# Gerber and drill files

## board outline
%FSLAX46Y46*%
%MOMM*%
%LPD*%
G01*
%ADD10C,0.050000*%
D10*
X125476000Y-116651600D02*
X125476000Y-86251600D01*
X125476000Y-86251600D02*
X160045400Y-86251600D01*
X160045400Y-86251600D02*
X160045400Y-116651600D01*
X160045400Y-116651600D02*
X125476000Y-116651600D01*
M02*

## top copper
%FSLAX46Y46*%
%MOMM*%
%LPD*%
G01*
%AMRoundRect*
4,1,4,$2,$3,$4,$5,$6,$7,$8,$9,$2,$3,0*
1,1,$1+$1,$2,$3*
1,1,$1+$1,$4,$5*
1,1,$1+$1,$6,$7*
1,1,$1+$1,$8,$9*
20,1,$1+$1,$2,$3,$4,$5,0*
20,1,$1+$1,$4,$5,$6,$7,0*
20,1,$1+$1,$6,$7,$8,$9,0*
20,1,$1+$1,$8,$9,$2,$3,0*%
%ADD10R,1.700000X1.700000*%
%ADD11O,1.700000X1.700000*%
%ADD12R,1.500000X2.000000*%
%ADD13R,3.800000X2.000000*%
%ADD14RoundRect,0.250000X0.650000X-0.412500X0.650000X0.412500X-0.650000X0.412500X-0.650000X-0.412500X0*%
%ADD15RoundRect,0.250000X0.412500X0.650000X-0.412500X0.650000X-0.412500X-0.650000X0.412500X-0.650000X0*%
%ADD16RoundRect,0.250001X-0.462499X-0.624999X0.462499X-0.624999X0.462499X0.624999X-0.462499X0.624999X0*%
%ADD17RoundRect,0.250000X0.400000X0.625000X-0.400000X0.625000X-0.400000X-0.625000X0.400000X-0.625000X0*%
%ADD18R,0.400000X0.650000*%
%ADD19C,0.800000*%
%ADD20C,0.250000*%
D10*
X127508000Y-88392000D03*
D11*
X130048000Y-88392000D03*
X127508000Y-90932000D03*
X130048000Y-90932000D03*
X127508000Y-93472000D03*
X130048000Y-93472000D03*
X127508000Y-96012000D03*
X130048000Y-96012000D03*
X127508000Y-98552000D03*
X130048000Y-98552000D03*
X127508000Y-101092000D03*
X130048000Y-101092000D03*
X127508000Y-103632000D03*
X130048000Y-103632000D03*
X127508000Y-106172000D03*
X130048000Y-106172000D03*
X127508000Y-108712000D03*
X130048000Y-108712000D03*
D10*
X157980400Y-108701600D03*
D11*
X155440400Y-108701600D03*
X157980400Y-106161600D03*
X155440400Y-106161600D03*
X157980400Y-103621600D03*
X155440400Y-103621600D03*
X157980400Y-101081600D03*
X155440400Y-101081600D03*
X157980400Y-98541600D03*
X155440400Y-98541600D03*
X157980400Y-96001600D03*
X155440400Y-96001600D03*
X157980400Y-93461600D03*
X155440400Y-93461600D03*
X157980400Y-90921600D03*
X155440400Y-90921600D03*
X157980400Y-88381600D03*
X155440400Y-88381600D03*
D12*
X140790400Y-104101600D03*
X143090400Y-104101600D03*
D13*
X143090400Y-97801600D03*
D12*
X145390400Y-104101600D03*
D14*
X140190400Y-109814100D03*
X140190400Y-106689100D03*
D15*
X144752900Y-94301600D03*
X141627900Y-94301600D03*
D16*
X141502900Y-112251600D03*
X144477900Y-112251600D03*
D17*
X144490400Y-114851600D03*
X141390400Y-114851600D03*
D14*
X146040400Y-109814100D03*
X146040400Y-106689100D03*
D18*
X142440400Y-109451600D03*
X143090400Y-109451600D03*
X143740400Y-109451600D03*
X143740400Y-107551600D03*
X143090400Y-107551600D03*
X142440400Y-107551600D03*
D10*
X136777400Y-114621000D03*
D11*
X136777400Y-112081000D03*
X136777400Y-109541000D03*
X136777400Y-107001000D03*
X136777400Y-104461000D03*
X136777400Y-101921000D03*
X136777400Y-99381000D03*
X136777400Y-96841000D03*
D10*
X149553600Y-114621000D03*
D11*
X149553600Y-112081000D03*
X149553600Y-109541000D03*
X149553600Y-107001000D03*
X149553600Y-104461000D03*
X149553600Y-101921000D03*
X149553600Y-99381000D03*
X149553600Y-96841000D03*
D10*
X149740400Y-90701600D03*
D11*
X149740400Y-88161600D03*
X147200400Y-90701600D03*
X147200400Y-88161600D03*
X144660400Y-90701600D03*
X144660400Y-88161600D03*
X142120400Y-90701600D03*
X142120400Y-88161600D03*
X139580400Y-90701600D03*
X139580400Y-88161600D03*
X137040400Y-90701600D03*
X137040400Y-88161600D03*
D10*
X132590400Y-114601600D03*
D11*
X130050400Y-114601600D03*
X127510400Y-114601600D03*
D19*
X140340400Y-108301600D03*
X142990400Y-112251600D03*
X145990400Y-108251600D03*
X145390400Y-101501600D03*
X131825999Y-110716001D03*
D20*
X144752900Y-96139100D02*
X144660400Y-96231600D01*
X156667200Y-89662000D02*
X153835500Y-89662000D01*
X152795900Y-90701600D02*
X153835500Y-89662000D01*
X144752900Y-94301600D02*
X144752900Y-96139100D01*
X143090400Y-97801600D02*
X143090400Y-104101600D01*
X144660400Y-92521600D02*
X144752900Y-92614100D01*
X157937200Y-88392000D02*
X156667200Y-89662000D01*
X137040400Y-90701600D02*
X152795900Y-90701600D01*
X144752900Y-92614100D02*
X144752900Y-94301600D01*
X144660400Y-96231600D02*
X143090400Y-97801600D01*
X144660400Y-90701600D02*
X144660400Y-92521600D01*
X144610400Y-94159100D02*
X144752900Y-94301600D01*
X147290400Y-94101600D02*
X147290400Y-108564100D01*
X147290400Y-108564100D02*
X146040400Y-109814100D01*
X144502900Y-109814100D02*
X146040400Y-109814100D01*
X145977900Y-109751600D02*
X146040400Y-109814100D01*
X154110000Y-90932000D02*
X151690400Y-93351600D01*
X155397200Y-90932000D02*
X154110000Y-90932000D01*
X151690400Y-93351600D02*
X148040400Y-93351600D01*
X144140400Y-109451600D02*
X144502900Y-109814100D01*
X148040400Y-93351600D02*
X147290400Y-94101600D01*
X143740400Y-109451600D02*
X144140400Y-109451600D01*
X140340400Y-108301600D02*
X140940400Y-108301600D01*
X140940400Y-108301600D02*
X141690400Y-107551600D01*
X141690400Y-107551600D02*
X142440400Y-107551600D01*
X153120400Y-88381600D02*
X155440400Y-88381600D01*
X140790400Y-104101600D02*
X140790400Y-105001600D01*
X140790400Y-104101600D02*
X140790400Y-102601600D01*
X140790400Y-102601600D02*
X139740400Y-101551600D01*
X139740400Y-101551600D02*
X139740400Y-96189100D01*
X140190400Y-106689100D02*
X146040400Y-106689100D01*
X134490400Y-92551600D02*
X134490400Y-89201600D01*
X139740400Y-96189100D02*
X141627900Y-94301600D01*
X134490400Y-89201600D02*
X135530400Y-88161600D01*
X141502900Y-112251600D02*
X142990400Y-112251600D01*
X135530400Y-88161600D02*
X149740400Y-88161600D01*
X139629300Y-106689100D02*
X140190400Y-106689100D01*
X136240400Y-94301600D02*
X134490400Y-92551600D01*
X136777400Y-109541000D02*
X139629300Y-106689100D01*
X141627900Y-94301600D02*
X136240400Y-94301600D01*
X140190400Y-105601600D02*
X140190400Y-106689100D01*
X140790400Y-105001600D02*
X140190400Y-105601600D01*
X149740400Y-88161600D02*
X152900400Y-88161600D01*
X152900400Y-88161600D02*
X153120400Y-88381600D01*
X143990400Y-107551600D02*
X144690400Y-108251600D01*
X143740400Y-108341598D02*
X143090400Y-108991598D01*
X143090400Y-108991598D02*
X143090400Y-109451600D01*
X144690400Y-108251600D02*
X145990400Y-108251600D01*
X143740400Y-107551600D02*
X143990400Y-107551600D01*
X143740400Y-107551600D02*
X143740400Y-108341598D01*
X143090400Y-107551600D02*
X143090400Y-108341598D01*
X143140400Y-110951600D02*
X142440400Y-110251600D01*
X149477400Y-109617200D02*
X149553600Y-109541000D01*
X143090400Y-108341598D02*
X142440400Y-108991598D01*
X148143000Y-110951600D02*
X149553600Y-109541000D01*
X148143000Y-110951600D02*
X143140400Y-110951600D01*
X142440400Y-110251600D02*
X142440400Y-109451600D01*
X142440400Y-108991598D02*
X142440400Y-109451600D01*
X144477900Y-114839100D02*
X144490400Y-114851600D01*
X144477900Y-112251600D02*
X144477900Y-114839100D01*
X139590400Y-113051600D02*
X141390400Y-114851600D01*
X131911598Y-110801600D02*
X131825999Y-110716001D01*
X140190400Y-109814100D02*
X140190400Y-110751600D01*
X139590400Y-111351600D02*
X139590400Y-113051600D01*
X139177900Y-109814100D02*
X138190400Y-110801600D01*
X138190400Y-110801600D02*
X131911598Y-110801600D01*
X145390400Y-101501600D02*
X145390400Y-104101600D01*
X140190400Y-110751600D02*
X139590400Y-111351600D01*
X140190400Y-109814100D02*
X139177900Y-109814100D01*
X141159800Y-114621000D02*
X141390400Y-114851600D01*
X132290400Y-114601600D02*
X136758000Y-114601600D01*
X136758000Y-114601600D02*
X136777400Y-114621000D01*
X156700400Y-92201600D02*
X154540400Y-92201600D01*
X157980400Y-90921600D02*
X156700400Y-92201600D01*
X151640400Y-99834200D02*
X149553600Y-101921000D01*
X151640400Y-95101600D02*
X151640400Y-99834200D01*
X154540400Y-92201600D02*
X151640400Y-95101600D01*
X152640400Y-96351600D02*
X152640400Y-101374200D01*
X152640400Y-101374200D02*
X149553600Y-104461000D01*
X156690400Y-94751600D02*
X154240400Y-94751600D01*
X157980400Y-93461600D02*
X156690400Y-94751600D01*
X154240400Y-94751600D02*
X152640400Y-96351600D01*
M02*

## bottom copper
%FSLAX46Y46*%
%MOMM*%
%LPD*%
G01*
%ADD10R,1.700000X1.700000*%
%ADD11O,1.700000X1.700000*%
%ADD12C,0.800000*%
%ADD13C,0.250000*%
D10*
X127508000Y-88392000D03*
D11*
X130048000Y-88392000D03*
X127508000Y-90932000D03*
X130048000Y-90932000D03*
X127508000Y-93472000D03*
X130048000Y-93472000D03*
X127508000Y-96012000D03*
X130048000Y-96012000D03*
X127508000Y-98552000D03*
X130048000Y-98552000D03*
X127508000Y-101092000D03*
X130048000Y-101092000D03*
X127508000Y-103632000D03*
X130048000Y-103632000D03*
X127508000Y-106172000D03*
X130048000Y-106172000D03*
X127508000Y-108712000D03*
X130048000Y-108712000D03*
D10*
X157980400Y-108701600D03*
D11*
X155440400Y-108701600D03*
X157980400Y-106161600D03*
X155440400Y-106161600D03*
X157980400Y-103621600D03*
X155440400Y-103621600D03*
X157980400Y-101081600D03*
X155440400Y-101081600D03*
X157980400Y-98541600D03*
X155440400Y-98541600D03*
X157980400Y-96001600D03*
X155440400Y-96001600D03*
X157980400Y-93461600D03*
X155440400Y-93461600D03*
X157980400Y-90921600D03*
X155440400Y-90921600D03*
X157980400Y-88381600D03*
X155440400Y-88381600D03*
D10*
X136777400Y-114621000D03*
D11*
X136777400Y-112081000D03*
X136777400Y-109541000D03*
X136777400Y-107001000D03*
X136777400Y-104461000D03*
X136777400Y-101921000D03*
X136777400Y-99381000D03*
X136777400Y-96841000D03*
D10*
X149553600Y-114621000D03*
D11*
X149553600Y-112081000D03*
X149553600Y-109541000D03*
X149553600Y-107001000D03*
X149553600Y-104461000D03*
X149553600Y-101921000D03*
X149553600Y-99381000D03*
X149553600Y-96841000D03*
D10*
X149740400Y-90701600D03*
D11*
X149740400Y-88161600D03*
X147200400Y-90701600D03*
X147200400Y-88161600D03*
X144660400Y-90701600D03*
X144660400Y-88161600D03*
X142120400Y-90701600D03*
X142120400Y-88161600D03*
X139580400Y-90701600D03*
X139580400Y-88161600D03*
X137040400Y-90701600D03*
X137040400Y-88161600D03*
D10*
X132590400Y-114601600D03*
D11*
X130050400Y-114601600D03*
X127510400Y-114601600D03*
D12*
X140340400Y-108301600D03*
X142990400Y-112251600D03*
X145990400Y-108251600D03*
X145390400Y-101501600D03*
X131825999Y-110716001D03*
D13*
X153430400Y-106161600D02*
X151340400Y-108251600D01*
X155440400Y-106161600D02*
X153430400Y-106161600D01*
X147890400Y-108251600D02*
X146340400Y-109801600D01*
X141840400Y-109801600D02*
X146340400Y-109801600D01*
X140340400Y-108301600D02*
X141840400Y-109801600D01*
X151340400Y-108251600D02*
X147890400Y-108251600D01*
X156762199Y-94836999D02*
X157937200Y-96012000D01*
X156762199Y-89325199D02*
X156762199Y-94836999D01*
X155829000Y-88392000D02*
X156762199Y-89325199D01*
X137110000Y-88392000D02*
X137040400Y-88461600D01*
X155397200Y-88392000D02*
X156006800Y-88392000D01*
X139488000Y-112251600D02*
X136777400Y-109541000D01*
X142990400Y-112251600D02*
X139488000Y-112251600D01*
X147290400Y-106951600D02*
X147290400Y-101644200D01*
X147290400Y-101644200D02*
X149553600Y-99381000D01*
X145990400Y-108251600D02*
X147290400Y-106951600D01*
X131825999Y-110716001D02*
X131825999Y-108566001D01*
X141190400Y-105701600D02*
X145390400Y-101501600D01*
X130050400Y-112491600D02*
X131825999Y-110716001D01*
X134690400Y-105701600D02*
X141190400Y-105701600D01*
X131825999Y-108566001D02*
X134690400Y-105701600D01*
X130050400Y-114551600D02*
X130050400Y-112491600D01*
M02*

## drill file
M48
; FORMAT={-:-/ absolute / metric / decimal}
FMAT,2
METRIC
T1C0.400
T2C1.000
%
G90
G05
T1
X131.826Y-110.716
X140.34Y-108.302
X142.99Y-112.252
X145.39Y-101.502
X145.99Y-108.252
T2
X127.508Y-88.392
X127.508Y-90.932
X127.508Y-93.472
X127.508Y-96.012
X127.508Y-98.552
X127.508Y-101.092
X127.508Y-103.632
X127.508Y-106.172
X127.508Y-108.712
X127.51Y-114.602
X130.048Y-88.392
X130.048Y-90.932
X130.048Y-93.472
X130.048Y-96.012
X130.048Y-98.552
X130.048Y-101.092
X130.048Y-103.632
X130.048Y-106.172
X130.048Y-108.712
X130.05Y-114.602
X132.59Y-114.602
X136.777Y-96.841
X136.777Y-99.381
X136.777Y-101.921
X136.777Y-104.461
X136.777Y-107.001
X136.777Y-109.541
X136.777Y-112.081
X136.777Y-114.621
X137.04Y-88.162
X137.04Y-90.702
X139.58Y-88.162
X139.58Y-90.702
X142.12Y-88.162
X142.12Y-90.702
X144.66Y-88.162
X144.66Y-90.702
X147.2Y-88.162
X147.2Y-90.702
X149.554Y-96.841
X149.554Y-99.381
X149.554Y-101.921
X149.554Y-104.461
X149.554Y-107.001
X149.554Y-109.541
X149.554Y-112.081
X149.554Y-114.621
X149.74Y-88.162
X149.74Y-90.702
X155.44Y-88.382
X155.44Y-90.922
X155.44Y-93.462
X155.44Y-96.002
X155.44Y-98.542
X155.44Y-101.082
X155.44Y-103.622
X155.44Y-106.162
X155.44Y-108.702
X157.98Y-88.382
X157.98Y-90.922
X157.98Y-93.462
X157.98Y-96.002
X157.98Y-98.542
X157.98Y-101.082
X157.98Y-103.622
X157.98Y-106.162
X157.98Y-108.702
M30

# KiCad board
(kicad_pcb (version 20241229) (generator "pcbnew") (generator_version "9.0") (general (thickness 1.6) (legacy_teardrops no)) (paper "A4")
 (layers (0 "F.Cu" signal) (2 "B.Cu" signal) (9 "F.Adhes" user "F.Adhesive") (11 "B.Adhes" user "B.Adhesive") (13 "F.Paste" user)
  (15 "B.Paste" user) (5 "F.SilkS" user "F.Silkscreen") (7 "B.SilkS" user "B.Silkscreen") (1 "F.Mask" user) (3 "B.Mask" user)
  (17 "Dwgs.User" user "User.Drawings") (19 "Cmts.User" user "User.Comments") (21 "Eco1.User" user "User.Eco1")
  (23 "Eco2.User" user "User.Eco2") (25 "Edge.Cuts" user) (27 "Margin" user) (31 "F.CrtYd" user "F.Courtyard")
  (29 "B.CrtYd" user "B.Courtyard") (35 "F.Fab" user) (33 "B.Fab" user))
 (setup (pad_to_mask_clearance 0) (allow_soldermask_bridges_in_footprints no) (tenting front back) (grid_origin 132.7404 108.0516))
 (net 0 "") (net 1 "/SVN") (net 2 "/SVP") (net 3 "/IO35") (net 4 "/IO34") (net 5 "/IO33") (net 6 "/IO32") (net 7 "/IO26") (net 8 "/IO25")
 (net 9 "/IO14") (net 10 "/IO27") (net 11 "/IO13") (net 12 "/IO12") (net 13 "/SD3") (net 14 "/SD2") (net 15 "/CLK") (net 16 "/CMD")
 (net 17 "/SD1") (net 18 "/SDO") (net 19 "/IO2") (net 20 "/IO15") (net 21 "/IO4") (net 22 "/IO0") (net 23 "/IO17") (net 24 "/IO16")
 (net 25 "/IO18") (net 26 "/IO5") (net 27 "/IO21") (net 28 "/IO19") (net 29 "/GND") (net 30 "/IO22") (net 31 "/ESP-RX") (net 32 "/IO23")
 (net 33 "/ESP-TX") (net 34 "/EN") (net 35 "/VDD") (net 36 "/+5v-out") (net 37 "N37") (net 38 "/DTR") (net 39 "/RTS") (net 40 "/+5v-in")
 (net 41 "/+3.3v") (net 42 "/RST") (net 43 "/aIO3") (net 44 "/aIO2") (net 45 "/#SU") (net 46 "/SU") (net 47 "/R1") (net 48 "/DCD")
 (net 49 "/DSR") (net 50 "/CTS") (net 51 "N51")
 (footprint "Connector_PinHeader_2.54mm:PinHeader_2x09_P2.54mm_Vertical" (layer "F.Cu") (at 127.508 88.392)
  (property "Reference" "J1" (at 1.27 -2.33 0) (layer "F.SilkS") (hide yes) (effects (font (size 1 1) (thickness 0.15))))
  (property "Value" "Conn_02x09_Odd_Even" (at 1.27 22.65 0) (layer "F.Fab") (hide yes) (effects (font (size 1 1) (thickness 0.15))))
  (pad "1" thru_hole rect (at 0 0) (size 1.7 1.7) (drill 1) (layers "*.Cu" "*.Mask") (remove_unused_layers no) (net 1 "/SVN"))
  (pad "2" thru_hole oval (at 2.54 0) (size 1.7 1.7) (drill 1) (layers "*.Cu" "*.Mask") (remove_unused_layers no) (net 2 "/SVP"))
  (pad "3" thru_hole oval (at 0 2.54) (size 1.7 1.7) (drill 1) (layers "*.Cu" "*.Mask") (remove_unused_layers no) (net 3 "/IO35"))
  (pad "4" thru_hole oval (at 2.54 2.54) (size 1.7 1.7) (drill 1) (layers "*.Cu" "*.Mask") (remove_unused_layers no) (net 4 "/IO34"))
  (pad "5" thru_hole oval (at 0 5.08) (size 1.7 1.7) (drill 1) (layers "*.Cu" "*.Mask") (remove_unused_layers no) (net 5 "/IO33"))
  (pad "6" thru_hole oval (at 2.54 5.08) (size 1.7 1.7) (drill 1) (layers "*.Cu" "*.Mask") (remove_unused_layers no) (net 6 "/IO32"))
  (pad "7" thru_hole oval (at 0 7.62) (size 1.7 1.7) (drill 1) (layers "*.Cu" "*.Mask") (remove_unused_layers no) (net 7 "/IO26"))
  (pad "8" thru_hole oval (at 2.54 7.62) (size 1.7 1.7) (drill 1) (layers "*.Cu" "*.Mask") (remove_unused_layers no) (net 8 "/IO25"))
  (pad "9" thru_hole oval (at 0 10.16) (size 1.7 1.7) (drill 1) (layers "*.Cu" "*.Mask") (remove_unused_layers no) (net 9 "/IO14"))
  (pad "10" thru_hole oval (at 2.54 10.16) (size 1.7 1.7) (drill 1) (layers "*.Cu" "*.Mask") (remove_unused_layers no) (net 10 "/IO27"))
  (pad "11" thru_hole oval (at 0 12.7) (size 1.7 1.7) (drill 1) (layers "*.Cu" "*.Mask") (remove_unused_layers no) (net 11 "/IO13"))
  (pad "12" thru_hole oval (at 2.54 12.7) (size 1.7 1.7) (drill 1) (layers "*.Cu" "*.Mask") (remove_unused_layers no) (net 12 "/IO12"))
  (pad "13" thru_hole oval (at 0 15.24) (size 1.7 1.7) (drill 1) (layers "*.Cu" "*.Mask") (remove_unused_layers no) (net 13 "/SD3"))
  (pad "14" thru_hole oval (at 2.54 15.24) (size 1.7 1.7) (drill 1) (layers "*.Cu" "*.Mask") (remove_unused_layers no) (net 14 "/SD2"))
  (pad "15" thru_hole oval (at 0 17.78) (size 1.7 1.7) (drill 1) (layers "*.Cu" "*.Mask") (remove_unused_layers no) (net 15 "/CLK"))
  (pad "16" thru_hole oval (at 2.54 17.78) (size 1.7 1.7) (drill 1) (layers "*.Cu" "*.Mask") (remove_unused_layers no) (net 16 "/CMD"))
  (pad "17" thru_hole oval (at 0 20.32) (size 1.7 1.7) (drill 1) (layers "*.Cu" "*.Mask") (remove_unused_layers no) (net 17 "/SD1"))
  (pad "18" thru_hole oval (at 2.54 20.32) (size 1.7 1.7) (drill 1) (layers "*.Cu" "*.Mask") (remove_unused_layers no) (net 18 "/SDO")))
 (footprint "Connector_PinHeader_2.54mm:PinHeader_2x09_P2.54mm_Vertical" (layer "F.Cu") (at 157.9804 108.7016 180)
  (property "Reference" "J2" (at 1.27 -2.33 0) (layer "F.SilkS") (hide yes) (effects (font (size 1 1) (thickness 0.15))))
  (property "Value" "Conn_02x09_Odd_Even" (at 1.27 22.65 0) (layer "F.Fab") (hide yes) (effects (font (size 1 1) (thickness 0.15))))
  (pad "1" thru_hole rect (at 0 0 180) (size 1.7 1.7) (drill 1) (layers "*.Cu" "*.Mask") (remove_unused_layers no) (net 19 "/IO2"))
  (pad "2" thru_hole oval (at 2.54 0 180) (size 1.7 1.7) (drill 1) (layers "*.Cu" "*.Mask") (remove_unused_layers no) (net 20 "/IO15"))
  (pad "3" thru_hole oval (at 0 2.54 180) (size 1.7 1.7) (drill 1) (layers "*.Cu" "*.Mask") (remove_unused_layers no) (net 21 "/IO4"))
  (pad "4" thru_hole oval (at 2.54 2.54 180) (size 1.7 1.7) (drill 1) (layers "*.Cu" "*.Mask") (remove_unused_layers no) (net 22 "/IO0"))
  (pad "5" thru_hole oval (at 0 5.08 180) (size 1.7 1.7) (drill 1) (layers "*.Cu" "*.Mask") (remove_unused_layers no) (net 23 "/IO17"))
  (pad "6" thru_hole oval (at 2.54 5.08 180) (size 1.7 1.7) (drill 1) (layers "*.Cu" "*.Mask") (remove_unused_layers no) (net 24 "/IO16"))
  (pad "7" thru_hole oval (at 0 7.62 180) (size 1.7 1.7) (drill 1) (layers "*.Cu" "*.Mask") (remove_unused_layers no) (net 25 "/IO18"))
  (pad "8" thru_hole oval (at 2.54 7.62 180) (size 1.7 1.7) (drill 1) (layers "*.Cu" "*.Mask") (remove_unused_layers no) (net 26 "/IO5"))
  (pad "9" thru_hole oval (at 0 10.16 180) (size 1.7 1.7) (drill 1) (layers "*.Cu" "*.Mask") (remove_unused_layers no) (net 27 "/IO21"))
  (pad "10" thru_hole oval (at 2.54 10.16 180) (size 1.7 1.7) (drill 1) (layers "*.Cu" "*.Mask") (remove_unused_layers no) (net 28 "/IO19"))
  (pad "11" thru_hole oval (at 0 12.7 180) (size 1.7 1.7) (drill 1) (layers "*.Cu" "*.Mask") (remove_unused_layers no) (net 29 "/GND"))
  (pad "12" thru_hole oval (at 2.54 12.7 180) (size 1.7 1.7) (drill 1) (layers "*.Cu" "*.Mask") (remove_unused_layers no) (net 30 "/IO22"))
  (pad "13" thru_hole oval (at 0 15.24 180) (size 1.7 1.7) (drill 1) (layers "*.Cu" "*.Mask") (remove_unused_layers no) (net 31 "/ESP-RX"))
  (pad "14" thru_hole oval (at 2.54 15.24 180) (size 1.7 1.7) (drill 1) (layers "*.Cu" "*.Mask") (remove_unused_layers no) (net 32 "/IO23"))
  (pad "15" thru_hole oval (at 0 17.78 180) (size 1.7 1.7) (drill 1) (layers "*.Cu" "*.Mask") (remove_unused_layers no) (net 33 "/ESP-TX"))
  (pad "16" thru_hole oval (at 2.54 17.78 180) (size 1.7 1.7) (drill 1) (layers "*.Cu" "*.Mask") (remove_unused_layers no) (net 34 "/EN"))
  (pad "17" thru_hole oval (at 0 20.32 180) (size 1.7 1.7) (drill 1) (layers "*.Cu" "*.Mask") (remove_unused_layers no) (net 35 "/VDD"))
  (pad "18" thru_hole oval (at 2.54 20.32 180) (size 1.7 1.7) (drill 1) (layers "*.Cu" "*.Mask") (remove_unused_layers no) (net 29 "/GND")))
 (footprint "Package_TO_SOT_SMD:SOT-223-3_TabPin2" (layer "F.Cu") (at 143.0904 100.9516 90)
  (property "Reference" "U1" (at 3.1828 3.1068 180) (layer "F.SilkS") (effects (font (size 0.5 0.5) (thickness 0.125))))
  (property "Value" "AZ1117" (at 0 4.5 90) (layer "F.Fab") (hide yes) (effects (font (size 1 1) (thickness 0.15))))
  (pad "1" smd rect (at -3.15 -2.3 90) (size 2 1.5) (layers "F.Cu" "F.Mask" "F.Paste") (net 29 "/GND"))
  (pad "2" smd rect (at -3.15 0 90) (size 2 1.5) (layers "F.Cu" "F.Mask" "F.Paste") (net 35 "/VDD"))
  (pad "2" smd rect (at 3.15 0 90) (size 2 3.8) (layers "F.Cu" "F.Mask" "F.Paste") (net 35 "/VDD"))
  (pad "3" smd rect (at -3.15 2.3 90) (size 2 1.5) (layers "F.Cu" "F.Mask" "F.Paste") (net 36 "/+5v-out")))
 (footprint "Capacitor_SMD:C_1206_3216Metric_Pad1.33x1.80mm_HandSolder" (layer "F.Cu") (at 140.1904 108.2516 90)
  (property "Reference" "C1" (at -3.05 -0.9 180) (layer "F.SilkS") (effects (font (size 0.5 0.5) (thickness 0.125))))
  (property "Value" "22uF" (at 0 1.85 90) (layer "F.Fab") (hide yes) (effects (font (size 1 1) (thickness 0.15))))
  (pad "1" smd roundrect (at -1.5625 0 90) (size 1.325 1.8) (layers "F.Cu" "F.Mask" "F.Paste") (roundrect_rratio 0.188679)
   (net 36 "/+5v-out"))
  (pad "2" smd roundrect (at 1.5625 0 90) (size 1.325 1.8) (layers "F.Cu" "F.Mask" "F.Paste") (roundrect_rratio 0.188679) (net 29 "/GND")))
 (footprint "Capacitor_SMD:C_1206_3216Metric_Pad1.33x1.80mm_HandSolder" (layer "F.Cu") (at 143.1904 94.3016 180)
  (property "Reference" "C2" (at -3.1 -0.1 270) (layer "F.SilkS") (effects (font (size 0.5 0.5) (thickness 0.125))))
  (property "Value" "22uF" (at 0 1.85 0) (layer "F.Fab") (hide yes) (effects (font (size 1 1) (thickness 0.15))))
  (pad "1" smd roundrect (at -1.5625 0 180) (size 1.325 1.8) (layers "F.Cu" "F.Mask" "F.Paste") (roundrect_rratio 0.188679) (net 35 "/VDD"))
  (pad "2" smd roundrect (at 1.5625 0 180) (size 1.325 1.8) (layers "F.Cu" "F.Mask" "F.Paste") (roundrect_rratio 0.188679) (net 29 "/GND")))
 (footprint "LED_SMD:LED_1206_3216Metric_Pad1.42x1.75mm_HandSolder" (layer "F.Cu") (at 142.9904 112.2516)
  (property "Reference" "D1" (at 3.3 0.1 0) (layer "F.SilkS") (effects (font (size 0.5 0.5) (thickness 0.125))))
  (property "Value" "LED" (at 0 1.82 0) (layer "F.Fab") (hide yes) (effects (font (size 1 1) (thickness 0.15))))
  (pad "1" smd roundrect (at -1.4875 0) (size 1.425 1.75) (layers "F.Cu" "F.Mask" "F.Paste") (roundrect_rratio 0.175439) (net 29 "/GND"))
  (pad "2" smd roundrect (at 1.4875 0) (size 1.425 1.75) (layers "F.Cu" "F.Mask" "F.Paste") (roundrect_rratio 0.175439) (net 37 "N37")))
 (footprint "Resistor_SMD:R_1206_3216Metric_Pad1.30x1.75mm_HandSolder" (layer "F.Cu") (at 142.9404 114.8516 180)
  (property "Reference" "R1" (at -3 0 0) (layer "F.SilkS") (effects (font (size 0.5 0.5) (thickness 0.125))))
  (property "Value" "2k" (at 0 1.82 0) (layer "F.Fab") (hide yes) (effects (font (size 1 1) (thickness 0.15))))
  (pad "1" smd roundrect (at -1.55 0 180) (size 1.3 1.75) (layers "F.Cu" "F.Mask" "F.Paste") (roundrect_rratio 0.192308) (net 37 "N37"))
  (pad "2" smd roundrect (at 1.55 0 180) (size 1.3 1.75) (layers "F.Cu" "F.Mask" "F.Paste") (roundrect_rratio 0.192308) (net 36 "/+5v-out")))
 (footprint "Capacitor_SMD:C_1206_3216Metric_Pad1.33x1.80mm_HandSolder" (layer "F.Cu") (at 146.0404 108.2516 90)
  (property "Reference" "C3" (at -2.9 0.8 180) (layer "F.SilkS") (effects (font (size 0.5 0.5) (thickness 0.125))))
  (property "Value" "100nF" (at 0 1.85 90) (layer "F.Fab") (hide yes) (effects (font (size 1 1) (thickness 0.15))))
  (pad "1" smd roundrect (at -1.5625 0 90) (size 1.325 1.8) (layers "F.Cu" "F.Mask" "F.Paste") (roundrect_rratio 0.188679) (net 34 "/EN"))
  (pad "2" smd roundrect (at 1.5625 0 90) (size 1.325 1.8) (layers "F.Cu" "F.Mask" "F.Paste") (roundrect_rratio 0.188679) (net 29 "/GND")))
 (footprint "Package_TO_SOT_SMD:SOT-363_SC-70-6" (layer "F.Cu") (at 143.0904 108.5016 90)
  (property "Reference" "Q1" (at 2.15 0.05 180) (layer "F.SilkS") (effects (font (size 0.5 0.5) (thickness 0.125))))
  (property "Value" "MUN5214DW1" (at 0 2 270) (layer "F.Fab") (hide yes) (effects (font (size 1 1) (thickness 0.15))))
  (pad "1" smd rect (at -0.95 -0.65 90) (size 0.65 0.4) (layers "F.Cu" "F.Mask" "F.Paste") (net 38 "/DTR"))
  (pad "2" smd rect (at -0.95 0 90) (size 0.65 0.4) (layers "F.Cu" "F.Mask" "F.Paste") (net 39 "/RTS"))
  (pad "3" smd rect (at -0.95 0.65 90) (size 0.65 0.4) (layers "F.Cu" "F.Mask" "F.Paste") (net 34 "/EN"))
  (pad "4" smd rect (at 0.95 0.65 90) (size 0.65 0.4) (layers "F.Cu" "F.Mask" "F.Paste") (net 39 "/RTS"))
  (pad "5" smd rect (at 0.95 0 90) (size 0.65 0.4) (layers "F.Cu" "F.Mask" "F.Paste") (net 38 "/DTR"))
  (pad "6" smd rect (at 0.95 -0.65 90) (size 0.65 0.4) (layers "F.Cu" "F.Mask" "F.Paste") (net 22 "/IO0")))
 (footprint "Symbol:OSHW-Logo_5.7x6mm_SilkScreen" (layer "B.Cu") (at 143.5404 95.6016 180)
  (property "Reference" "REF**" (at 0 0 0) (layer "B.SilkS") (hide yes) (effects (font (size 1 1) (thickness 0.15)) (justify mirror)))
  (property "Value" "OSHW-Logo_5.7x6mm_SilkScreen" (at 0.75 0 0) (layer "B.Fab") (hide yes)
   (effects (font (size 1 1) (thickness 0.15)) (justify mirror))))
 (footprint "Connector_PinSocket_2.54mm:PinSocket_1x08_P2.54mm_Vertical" (layer "B.Cu") (at 136.7774 114.621)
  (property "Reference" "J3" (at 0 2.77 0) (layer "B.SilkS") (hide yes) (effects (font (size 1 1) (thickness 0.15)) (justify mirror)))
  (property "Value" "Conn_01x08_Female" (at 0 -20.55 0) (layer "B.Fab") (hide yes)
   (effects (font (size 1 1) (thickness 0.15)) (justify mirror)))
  (pad "1" thru_hole rect (at 0 0) (size 1.7 1.7) (drill 1) (layers "*.Cu" "*.Mask") (remove_unused_layers no) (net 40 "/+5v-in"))
  (pad "2" thru_hole oval (at 0 -2.54) (size 1.7 1.7) (drill 1) (layers "*.Cu" "*.Mask") (remove_unused_layers no) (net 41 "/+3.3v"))
  (pad "3" thru_hole oval (at 0 -5.08) (size 1.7 1.7) (drill 1) (layers "*.Cu" "*.Mask") (remove_unused_layers no) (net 29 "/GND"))
  (pad "4" thru_hole oval (at 0 -7.62) (size 1.7 1.7) (drill 1) (layers "*.Cu" "*.Mask") (remove_unused_layers no) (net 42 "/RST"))
  (pad "5" thru_hole oval (at 0 -10.16) (size 1.7 1.7) (drill 1) (layers "*.Cu" "*.Mask") (remove_unused_layers no) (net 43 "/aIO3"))
  (pad "6" thru_hole oval (at 0 -12.7) (size 1.7 1.7) (drill 1) (layers "*.Cu" "*.Mask") (remove_unused_layers no) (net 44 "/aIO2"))
  (pad "7" thru_hole oval (at 0 -15.24) (size 1.7 1.7) (drill 1) (layers "*.Cu" "*.Mask") (remove_unused_layers no) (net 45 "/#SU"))
  (pad "8" thru_hole oval (at 0 -17.78) (size 1.7 1.7) (drill 1) (layers "*.Cu" "*.Mask") (remove_unused_layers no) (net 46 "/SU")))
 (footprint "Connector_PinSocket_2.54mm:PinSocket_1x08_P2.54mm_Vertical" (layer "B.Cu") (at 149.5536 114.621)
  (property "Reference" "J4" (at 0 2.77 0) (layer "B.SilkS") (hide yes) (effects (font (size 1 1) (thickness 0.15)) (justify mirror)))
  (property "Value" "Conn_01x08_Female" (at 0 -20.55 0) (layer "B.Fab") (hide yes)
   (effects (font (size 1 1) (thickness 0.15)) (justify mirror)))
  (pad "1" thru_hole rect (at 0 0) (size 1.7 1.7) (drill 1) (layers "*.Cu" "*.Mask") (remove_unused_layers no) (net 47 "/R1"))
  (pad "2" thru_hole oval (at 0 -2.54) (size 1.7 1.7) (drill 1) (layers "*.Cu" "*.Mask") (remove_unused_layers no) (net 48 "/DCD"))
  (pad "3" thru_hole oval (at 0 -5.08) (size 1.7 1.7) (drill 1) (layers "*.Cu" "*.Mask") (remove_unused_layers no) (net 38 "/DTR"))
  (pad "4" thru_hole oval (at 0 -7.62) (size 1.7 1.7) (drill 1) (layers "*.Cu" "*.Mask") (remove_unused_layers no) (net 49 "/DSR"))
  (pad "5" thru_hole oval (at 0 -10.16) (size 1.7 1.7) (drill 1) (layers "*.Cu" "*.Mask") (remove_unused_layers no) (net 31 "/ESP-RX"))
  (pad "6" thru_hole oval (at 0 -12.7) (size 1.7 1.7) (drill 1) (layers "*.Cu" "*.Mask") (remove_unused_layers no) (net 33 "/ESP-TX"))
  (pad "7" thru_hole oval (at 0 -15.24) (size 1.7 1.7) (drill 1) (layers "*.Cu" "*.Mask") (remove_unused_layers no) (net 39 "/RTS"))
  (pad "8" thru_hole oval (at 0 -17.78) (size 1.7 1.7) (drill 1) (layers "*.Cu" "*.Mask") (remove_unused_layers no) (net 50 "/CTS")))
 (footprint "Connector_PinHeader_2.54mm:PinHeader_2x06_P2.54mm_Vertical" (layer "B.Cu") (at 149.7404 90.7016 90)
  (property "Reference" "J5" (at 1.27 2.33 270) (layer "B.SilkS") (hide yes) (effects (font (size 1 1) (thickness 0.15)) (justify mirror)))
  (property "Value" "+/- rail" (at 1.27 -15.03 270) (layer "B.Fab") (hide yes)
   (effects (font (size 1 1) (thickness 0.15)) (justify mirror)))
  (pad "1" thru_hole rect (at 0 0 90) (size 1.7 1.7) (drill 1) (layers "*.Cu" "*.Mask") (remove_unused_layers no) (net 35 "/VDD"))
  (pad "2" thru_hole oval (at 2.54 0 90) (size 1.7 1.7) (drill 1) (layers "*.Cu" "*.Mask") (remove_unused_layers no) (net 29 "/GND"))
  (pad "3" thru_hole oval (at 0 -2.54 90) (size 1.7 1.7) (drill 1) (layers "*.Cu" "*.Mask") (remove_unused_layers no) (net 35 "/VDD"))
  (pad "4" thru_hole oval (at 2.54 -2.54 90) (size 1.7 1.7) (drill 1) (layers "*.Cu" "*.Mask") (remove_unused_layers no) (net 29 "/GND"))
  (pad "5" thru_hole oval (at 0 -5.08 90) (size 1.7 1.7) (drill 1) (layers "*.Cu" "*.Mask") (remove_unused_layers no) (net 35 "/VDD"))
  (pad "6" thru_hole oval (at 2.54 -5.08 90) (size 1.7 1.7) (drill 1) (layers "*.Cu" "*.Mask") (remove_unused_layers no) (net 29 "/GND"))
  (pad "7" thru_hole oval (at 0 -7.62 90) (size 1.7 1.7) (drill 1) (layers "*.Cu" "*.Mask") (remove_unused_layers no) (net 35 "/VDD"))
  (pad "8" thru_hole oval (at 2.54 -7.62 90) (size 1.7 1.7) (drill 1) (layers "*.Cu" "*.Mask") (remove_unused_layers no) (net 29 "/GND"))
  (pad "9" thru_hole oval (at 0 -10.16 90) (size 1.7 1.7) (drill 1) (layers "*.Cu" "*.Mask") (remove_unused_layers no) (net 35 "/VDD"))
  (pad "10" thru_hole oval (at 2.54 -10.16 90) (size 1.7 1.7) (drill 1) (layers "*.Cu" "*.Mask") (remove_unused_layers no) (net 29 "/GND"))
  (pad "11" thru_hole oval (at 0 -12.7 90) (size 1.7 1.7) (drill 1) (layers "*.Cu" "*.Mask") (remove_unused_layers no) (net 35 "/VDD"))
  (pad "12" thru_hole oval (at 2.54 -12.7 90) (size 1.7 1.7) (drill 1) (layers "*.Cu" "*.Mask") (remove_unused_layers no) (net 29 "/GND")))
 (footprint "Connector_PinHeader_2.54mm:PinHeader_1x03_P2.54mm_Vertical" (layer "B.Cu") (at 132.5904 114.6016 90)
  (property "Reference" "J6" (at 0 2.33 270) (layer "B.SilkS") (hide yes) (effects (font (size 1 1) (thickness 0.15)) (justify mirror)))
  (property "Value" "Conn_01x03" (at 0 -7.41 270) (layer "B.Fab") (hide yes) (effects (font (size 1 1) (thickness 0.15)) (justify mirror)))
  (pad "1" thru_hole rect (at 0 0 90) (size 1.7 1.7) (drill 1) (layers "*.Cu" "*.Mask") (remove_unused_layers no) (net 40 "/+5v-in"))
  (pad "2" thru_hole oval (at 0 -2.54 90) (size 1.7 1.7) (drill 1) (layers "*.Cu" "*.Mask") (remove_unused_layers no) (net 36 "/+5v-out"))
  (pad "3" thru_hole oval (at 0 -5.08 90) (size 1.7 1.7) (drill 1) (layers "*.Cu" "*.Mask") (remove_unused_layers no) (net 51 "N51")))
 (gr_line (start 125.476 116.6516) (end 125.476 86.2516) (stroke (width 0.05) (type solid)) (layer "Edge.Cuts"))
 (gr_line (start 125.476 86.2516) (end 160.0454 86.2516) (stroke (width 0.05) (type solid)) (layer "Edge.Cuts"))
 (gr_line (start 160.0454 86.2516) (end 160.0454 116.6516) (stroke (width 0.05) (type solid)) (layer "Edge.Cuts"))
 (gr_line (start 160.0454 116.6516) (end 125.476 116.6516) (stroke (width 0.05) (type solid)) (layer "Edge.Cuts"))
 (segment (start 144.7529 96.1391) (end 144.6604 96.2316) (width 0.25) (layer "F.Cu") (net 35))
 (segment (start 156.6672 89.662) (end 153.8355 89.662) (width 0.25) (layer "F.Cu") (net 35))
 (segment (start 152.7959 90.7016) (end 153.8355 89.662) (width 0.25) (layer "F.Cu") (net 35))
 (segment (start 144.7529 94.3016) (end 144.7529 96.1391) (width 0.25) (layer "F.Cu") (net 35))
 (segment (start 143.0904 97.8016) (end 143.0904 104.1016) (width 0.25) (layer "F.Cu") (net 35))
 (segment (start 144.6604 92.5216) (end 144.7529 92.6141) (width 0.25) (layer "F.Cu") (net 35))
 (segment (start 157.9372 88.392) (end 156.6672 89.662) (width 0.25) (layer "F.Cu") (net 35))
 (segment (start 137.0404 90.7016) (end 152.7959 90.7016) (width 0.25) (layer "F.Cu") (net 35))
 (segment (start 144.7529 92.6141) (end 144.7529 94.3016) (width 0.25) (layer "F.Cu") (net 35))
 (segment (start 144.6604 96.2316) (end 143.0904 97.8016) (width 0.25) (layer "F.Cu") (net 35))
 (segment (start 144.6604 90.7016) (end 144.6604 92.5216) (width 0.25) (layer "F.Cu") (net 35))
 (segment (start 144.6104 94.1591) (end 144.7529 94.3016) (width 0.25) (layer "F.Cu") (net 35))
 (segment (start 147.2904 94.1016) (end 147.2904 108.5641) (width 0.25) (layer "F.Cu") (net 34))
 (segment (start 147.2904 108.5641) (end 146.0404 109.8141) (width 0.25) (layer "F.Cu") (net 34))
 (segment (start 144.5029 109.8141) (end 146.0404 109.8141) (width 0.25) (layer "F.Cu") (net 34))
 (segment (start 145.9779 109.7516) (end 146.0404 109.8141) (width 0.25) (layer "F.Cu") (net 34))
 (segment (start 154.11 90.932) (end 151.6904 93.3516) (width 0.25) (layer "F.Cu") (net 34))
 (segment (start 155.3972 90.932) (end 154.11 90.932) (width 0.25) (layer "F.Cu") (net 34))
 (segment (start 151.6904 93.3516) (end 148.0404 93.3516) (width 0.25) (layer "F.Cu") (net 34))
 (segment (start 144.1404 109.4516) (end 144.5029 109.8141) (width 0.25) (layer "F.Cu") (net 34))
 (segment (start 148.0404 93.3516) (end 147.2904 94.1016) (width 0.25) (layer "F.Cu") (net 34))
 (segment (start 143.7404 109.4516) (end 144.1404 109.4516) (width 0.25) (layer "F.Cu") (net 34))
 (segment (start 140.3404 108.3016) (end 140.9404 108.3016) (width 0.25) (layer "F.Cu") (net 22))
 (segment (start 140.9404 108.3016) (end 141.6904 107.5516) (width 0.25) (layer "F.Cu") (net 22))
 (segment (start 141.6904 107.5516) (end 142.4404 107.5516) (width 0.25) (layer "F.Cu") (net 22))
 (via (at 140.3404 108.3016) (size 0.8) (drill 0.4) (layers "F.Cu" "B.Cu") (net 22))
 (segment (start 153.4304 106.1616) (end 151.3404 108.2516) (width 0.25) (layer "B.Cu") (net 22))
 (segment (start 155.4404 106.1616) (end 153.4304 106.1616) (width 0.25) (layer "B.Cu") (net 22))
 (segment (start 147.8904 108.2516) (end 146.3404 109.8016) (width 0.25) (layer "B.Cu") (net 22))
 (segment (start 141.8404 109.8016) (end 146.3404 109.8016) (width 0.25) (layer "B.Cu") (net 22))
 (segment (start 140.3404 108.3016) (end 141.8404 109.8016) (width 0.25) (layer "B.Cu") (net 22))
 (segment (start 151.3404 108.2516) (end 147.8904 108.2516) (width 0.25) (layer "B.Cu") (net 22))
 (segment (start 153.1204 88.3816) (end 155.4404 88.3816) (width 0.25) (layer "F.Cu") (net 29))
 (segment (start 140.7904 104.1016) (end 140.7904 105.0016) (width 0.25) (layer "F.Cu") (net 29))
 (segment (start 140.7904 104.1016) (end 140.7904 102.6016) (width 0.25) (layer "F.Cu") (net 29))
 (segment (start 140.7904 102.6016) (end 139.7404 101.5516) (width 0.25) (layer "F.Cu") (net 29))
 (segment (start 139.7404 101.5516) (end 139.7404 96.1891) (width 0.25) (layer "F.Cu") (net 29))
 (segment (start 140.1904 106.6891) (end 146.0404 106.6891) (width 0.25) (layer "F.Cu") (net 29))
 (segment (start 134.4904 92.5516) (end 134.4904 89.2016) (width 0.25) (layer "F.Cu") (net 29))
 (segment (start 139.7404 96.1891) (end 141.6279 94.3016) (width 0.25) (layer "F.Cu") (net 29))
 (segment (start 134.4904 89.2016) (end 135.5304 88.1616) (width 0.25) (layer "F.Cu") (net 29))
 (segment (start 141.5029 112.2516) (end 142.9904 112.2516) (width 0.25) (layer "F.Cu") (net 29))
 (segment (start 135.5304 88.1616) (end 149.7404 88.1616) (width 0.25) (layer "F.Cu") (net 29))
 (segment (start 139.6293 106.6891) (end 140.1904 106.6891) (width 0.25) (layer "F.Cu") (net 29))
 (segment (start 136.2404 94.3016) (end 134.4904 92.5516) (width 0.25) (layer "F.Cu") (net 29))
 (segment (start 136.7774 109.541) (end 139.6293 106.6891) (width 0.25) (layer "F.Cu") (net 29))
 (segment (start 141.6279 94.3016) (end 136.2404 94.3016) (width 0.25) (layer "F.Cu") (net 29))
 (segment (start 140.1904 105.6016) (end 140.1904 106.6891) (width 0.25) (layer "F.Cu") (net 29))
 (segment (start 140.7904 105.0016) (end 140.1904 105.6016) (width 0.25) (layer "F.Cu") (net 29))
 (segment (start 149.7404 88.1616) (end 152.9004 88.1616) (width 0.25) (layer "F.Cu") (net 29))
 (segment (start 152.9004 88.1616) (end 153.1204 88.3816) (width 0.25) (layer "F.Cu") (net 29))
 (via (at 142.9904 112.2516) (size 0.8) (drill 0.4) (layers "F.Cu" "B.Cu") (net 29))
 (segment (start 156.762199 94.836999) (end 157.9372 96.012) (width 0.25) (layer "B.Cu") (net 29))
 (segment (start 156.762199 89.325199) (end 156.762199 94.836999) (width 0.25) (layer "B.Cu") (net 29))
 (segment (start 155.829 88.392) (end 156.762199 89.325199) (width 0.25) (layer "B.Cu") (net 29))
 (segment (start 137.11 88.392) (end 137.0404 88.4616) (width 0.25) (layer "B.Cu") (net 29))
 (segment (start 155.3972 88.392) (end 156.0068 88.392) (width 0.25) (layer "B.Cu") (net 29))
 (segment (start 139.488 112.2516) (end 136.7774 109.541) (width 0.25) (layer "B.Cu") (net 29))
 (segment (start 142.9904 112.2516) (end 139.488 112.2516) (width 0.25) (layer "B.Cu") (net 29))
 (segment (start 143.9904 107.5516) (end 144.6904 108.2516) (width 0.25) (layer "F.Cu") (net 39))
 (segment (start 143.7404 108.341598) (end 143.0904 108.991598) (width 0.25) (layer "F.Cu") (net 39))
 (segment (start 143.0904 108.991598) (end 143.0904 109.4516) (width 0.25) (layer "F.Cu") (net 39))
 (segment (start 144.6904 108.2516) (end 145.9904 108.2516) (width 0.25) (layer "F.Cu") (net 39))
 (segment (start 143.7404 107.5516) (end 143.9904 107.5516) (width 0.25) (layer "F.Cu") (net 39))
 (segment (start 143.7404 107.5516) (end 143.7404 108.341598) (width 0.25) (layer "F.Cu") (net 39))
 (via (at 145.9904 108.2516) (size 0.8) (drill 0.4) (layers "F.Cu" "B.Cu") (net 39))
 (segment (start 147.2904 106.9516) (end 147.2904 101.6442) (width 0.25) (layer "B.Cu") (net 39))
 (segment (start 147.2904 101.6442) (end 149.5536 99.381) (width 0.25) (layer "B.Cu") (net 39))
 (segment (start 145.9904 108.2516) (end 147.2904 106.9516) (width 0.25) (layer "B.Cu") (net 39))
 (segment (start 143.0904 107.5516) (end 143.0904 108.341598) (width 0.25) (layer "F.Cu") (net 38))
 (segment (start 143.1404 110.9516) (end 142.4404 110.2516) (width 0.25) (layer "F.Cu") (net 38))
 (segment (start 149.4774 109.6172) (end 149.5536 109.541) (width 0.25) (layer "F.Cu") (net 38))
 (segment (start 143.0904 108.341598) (end 142.4404 108.991598) (width 0.25) (layer "F.Cu") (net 38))
 (segment (start 148.143 110.9516) (end 149.5536 109.541) (width 0.25) (layer "F.Cu") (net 38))
 (segment (start 148.143 110.9516) (end 143.1404 110.9516) (width 0.25) (layer "F.Cu") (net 38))
 (segment (start 142.4404 110.2516) (end 142.4404 109.4516) (width 0.25) (layer "F.Cu") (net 38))
 (segment (start 142.4404 108.991598) (end 142.4404 109.4516) (width 0.25) (layer "F.Cu") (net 38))
 (segment (start 144.4779 114.8391) (end 144.4904 114.8516) (width 0.25) (layer "F.Cu") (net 37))
 (segment (start 144.4779 112.2516) (end 144.4779 114.8391) (width 0.25) (layer "F.Cu") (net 37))
 (segment (start 139.5904 113.0516) (end 141.3904 114.8516) (width 0.25) (layer "F.Cu") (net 36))
 (segment (start 131.911598 110.8016) (end 131.825999 110.716001) (width 0.25) (layer "F.Cu") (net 36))
 (segment (start 140.1904 109.8141) (end 140.1904 110.7516) (width 0.25) (layer "F.Cu") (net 36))
 (segment (start 139.5904 111.3516) (end 139.5904 113.0516) (width 0.25) (layer "F.Cu") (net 36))
 (segment (start 139.1779 109.8141) (end 138.1904 110.8016) (width 0.25) (layer "F.Cu") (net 36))
 (segment (start 138.1904 110.8016) (end 131.911598 110.8016) (width 0.25) (layer "F.Cu") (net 36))
 (segment (start 145.3904 101.5016) (end 145.3904 104.1016) (width 0.25) (layer "F.Cu") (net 36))
 (segment (start 140.1904 110.7516) (end 139.5904 111.3516) (width 0.25) (layer "F.Cu") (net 36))
 (segment (start 140.1904 109.8141) (end 139.1779 109.8141) (width 0.25) (layer "F.Cu") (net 36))
 (segment (start 141.1598 114.621) (end 141.3904 114.8516) (width 0.25) (layer "F.Cu") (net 36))
 (via (at 145.3904 101.5016) (size 0.8) (drill 0.4) (layers "F.Cu" "B.Cu") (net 36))
 (via (at 131.825999 110.716001) (size 0.8) (drill 0.4) (layers "F.Cu" "B.Cu") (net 36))
 (segment (start 131.825999 110.716001) (end 131.825999 108.566001) (width 0.25) (layer "B.Cu") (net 36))
 (segment (start 141.1904 105.7016) (end 145.3904 101.5016) (width 0.25) (layer "B.Cu") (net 36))
 (segment (start 130.0504 112.4916) (end 131.825999 110.716001) (width 0.25) (layer "B.Cu") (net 36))
 (segment (start 134.6904 105.7016) (end 141.1904 105.7016) (width 0.25) (layer "B.Cu") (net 36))
 (segment (start 131.825999 108.566001) (end 134.6904 105.7016) (width 0.25) (layer "B.Cu") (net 36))
 (segment (start 130.0504 114.5516) (end 130.0504 112.4916) (width 0.25) (layer "B.Cu") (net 36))
 (segment (start 132.2904 114.6016) (end 136.758 114.6016) (width 0.25) (layer "F.Cu") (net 40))
 (segment (start 136.758 114.6016) (end 136.7774 114.621) (width 0.25) (layer "F.Cu") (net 40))
 (segment (start 156.7004 92.2016) (end 154.5404 92.2016) (width 0.25) (layer "F.Cu") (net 33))
 (segment (start 157.9804 90.9216) (end 156.7004 92.2016) (width 0.25) (layer "F.Cu") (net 33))
 (segment (start 151.6404 99.8342) (end 149.5536 101.921) (width 0.25) (layer "F.Cu") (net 33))
 (segment (start 151.6404 95.1016) (end 151.6404 99.8342) (width 0.25) (layer "F.Cu") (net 33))
 (segment (start 154.5404 92.2016) (end 151.6404 95.1016) (width 0.25) (layer "F.Cu") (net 33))
 (segment (start 152.6404 96.3516) (end 152.6404 101.3742) (width 0.25) (layer "F.Cu") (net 31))
 (segment (start 152.6404 101.3742) (end 149.5536 104.461) (width 0.25) (layer "F.Cu") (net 31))
 (segment (start 156.6904 94.7516) (end 154.2404 94.7516) (width 0.25) (layer "F.Cu") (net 31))
 (segment (start 157.9804 93.4616) (end 156.6904 94.7516) (width 0.25) (layer "F.Cu") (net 31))
 (segment (start 154.2404 94.7516) (end 152.6404 96.3516) (width 0.25) (layer "F.Cu") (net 31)))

